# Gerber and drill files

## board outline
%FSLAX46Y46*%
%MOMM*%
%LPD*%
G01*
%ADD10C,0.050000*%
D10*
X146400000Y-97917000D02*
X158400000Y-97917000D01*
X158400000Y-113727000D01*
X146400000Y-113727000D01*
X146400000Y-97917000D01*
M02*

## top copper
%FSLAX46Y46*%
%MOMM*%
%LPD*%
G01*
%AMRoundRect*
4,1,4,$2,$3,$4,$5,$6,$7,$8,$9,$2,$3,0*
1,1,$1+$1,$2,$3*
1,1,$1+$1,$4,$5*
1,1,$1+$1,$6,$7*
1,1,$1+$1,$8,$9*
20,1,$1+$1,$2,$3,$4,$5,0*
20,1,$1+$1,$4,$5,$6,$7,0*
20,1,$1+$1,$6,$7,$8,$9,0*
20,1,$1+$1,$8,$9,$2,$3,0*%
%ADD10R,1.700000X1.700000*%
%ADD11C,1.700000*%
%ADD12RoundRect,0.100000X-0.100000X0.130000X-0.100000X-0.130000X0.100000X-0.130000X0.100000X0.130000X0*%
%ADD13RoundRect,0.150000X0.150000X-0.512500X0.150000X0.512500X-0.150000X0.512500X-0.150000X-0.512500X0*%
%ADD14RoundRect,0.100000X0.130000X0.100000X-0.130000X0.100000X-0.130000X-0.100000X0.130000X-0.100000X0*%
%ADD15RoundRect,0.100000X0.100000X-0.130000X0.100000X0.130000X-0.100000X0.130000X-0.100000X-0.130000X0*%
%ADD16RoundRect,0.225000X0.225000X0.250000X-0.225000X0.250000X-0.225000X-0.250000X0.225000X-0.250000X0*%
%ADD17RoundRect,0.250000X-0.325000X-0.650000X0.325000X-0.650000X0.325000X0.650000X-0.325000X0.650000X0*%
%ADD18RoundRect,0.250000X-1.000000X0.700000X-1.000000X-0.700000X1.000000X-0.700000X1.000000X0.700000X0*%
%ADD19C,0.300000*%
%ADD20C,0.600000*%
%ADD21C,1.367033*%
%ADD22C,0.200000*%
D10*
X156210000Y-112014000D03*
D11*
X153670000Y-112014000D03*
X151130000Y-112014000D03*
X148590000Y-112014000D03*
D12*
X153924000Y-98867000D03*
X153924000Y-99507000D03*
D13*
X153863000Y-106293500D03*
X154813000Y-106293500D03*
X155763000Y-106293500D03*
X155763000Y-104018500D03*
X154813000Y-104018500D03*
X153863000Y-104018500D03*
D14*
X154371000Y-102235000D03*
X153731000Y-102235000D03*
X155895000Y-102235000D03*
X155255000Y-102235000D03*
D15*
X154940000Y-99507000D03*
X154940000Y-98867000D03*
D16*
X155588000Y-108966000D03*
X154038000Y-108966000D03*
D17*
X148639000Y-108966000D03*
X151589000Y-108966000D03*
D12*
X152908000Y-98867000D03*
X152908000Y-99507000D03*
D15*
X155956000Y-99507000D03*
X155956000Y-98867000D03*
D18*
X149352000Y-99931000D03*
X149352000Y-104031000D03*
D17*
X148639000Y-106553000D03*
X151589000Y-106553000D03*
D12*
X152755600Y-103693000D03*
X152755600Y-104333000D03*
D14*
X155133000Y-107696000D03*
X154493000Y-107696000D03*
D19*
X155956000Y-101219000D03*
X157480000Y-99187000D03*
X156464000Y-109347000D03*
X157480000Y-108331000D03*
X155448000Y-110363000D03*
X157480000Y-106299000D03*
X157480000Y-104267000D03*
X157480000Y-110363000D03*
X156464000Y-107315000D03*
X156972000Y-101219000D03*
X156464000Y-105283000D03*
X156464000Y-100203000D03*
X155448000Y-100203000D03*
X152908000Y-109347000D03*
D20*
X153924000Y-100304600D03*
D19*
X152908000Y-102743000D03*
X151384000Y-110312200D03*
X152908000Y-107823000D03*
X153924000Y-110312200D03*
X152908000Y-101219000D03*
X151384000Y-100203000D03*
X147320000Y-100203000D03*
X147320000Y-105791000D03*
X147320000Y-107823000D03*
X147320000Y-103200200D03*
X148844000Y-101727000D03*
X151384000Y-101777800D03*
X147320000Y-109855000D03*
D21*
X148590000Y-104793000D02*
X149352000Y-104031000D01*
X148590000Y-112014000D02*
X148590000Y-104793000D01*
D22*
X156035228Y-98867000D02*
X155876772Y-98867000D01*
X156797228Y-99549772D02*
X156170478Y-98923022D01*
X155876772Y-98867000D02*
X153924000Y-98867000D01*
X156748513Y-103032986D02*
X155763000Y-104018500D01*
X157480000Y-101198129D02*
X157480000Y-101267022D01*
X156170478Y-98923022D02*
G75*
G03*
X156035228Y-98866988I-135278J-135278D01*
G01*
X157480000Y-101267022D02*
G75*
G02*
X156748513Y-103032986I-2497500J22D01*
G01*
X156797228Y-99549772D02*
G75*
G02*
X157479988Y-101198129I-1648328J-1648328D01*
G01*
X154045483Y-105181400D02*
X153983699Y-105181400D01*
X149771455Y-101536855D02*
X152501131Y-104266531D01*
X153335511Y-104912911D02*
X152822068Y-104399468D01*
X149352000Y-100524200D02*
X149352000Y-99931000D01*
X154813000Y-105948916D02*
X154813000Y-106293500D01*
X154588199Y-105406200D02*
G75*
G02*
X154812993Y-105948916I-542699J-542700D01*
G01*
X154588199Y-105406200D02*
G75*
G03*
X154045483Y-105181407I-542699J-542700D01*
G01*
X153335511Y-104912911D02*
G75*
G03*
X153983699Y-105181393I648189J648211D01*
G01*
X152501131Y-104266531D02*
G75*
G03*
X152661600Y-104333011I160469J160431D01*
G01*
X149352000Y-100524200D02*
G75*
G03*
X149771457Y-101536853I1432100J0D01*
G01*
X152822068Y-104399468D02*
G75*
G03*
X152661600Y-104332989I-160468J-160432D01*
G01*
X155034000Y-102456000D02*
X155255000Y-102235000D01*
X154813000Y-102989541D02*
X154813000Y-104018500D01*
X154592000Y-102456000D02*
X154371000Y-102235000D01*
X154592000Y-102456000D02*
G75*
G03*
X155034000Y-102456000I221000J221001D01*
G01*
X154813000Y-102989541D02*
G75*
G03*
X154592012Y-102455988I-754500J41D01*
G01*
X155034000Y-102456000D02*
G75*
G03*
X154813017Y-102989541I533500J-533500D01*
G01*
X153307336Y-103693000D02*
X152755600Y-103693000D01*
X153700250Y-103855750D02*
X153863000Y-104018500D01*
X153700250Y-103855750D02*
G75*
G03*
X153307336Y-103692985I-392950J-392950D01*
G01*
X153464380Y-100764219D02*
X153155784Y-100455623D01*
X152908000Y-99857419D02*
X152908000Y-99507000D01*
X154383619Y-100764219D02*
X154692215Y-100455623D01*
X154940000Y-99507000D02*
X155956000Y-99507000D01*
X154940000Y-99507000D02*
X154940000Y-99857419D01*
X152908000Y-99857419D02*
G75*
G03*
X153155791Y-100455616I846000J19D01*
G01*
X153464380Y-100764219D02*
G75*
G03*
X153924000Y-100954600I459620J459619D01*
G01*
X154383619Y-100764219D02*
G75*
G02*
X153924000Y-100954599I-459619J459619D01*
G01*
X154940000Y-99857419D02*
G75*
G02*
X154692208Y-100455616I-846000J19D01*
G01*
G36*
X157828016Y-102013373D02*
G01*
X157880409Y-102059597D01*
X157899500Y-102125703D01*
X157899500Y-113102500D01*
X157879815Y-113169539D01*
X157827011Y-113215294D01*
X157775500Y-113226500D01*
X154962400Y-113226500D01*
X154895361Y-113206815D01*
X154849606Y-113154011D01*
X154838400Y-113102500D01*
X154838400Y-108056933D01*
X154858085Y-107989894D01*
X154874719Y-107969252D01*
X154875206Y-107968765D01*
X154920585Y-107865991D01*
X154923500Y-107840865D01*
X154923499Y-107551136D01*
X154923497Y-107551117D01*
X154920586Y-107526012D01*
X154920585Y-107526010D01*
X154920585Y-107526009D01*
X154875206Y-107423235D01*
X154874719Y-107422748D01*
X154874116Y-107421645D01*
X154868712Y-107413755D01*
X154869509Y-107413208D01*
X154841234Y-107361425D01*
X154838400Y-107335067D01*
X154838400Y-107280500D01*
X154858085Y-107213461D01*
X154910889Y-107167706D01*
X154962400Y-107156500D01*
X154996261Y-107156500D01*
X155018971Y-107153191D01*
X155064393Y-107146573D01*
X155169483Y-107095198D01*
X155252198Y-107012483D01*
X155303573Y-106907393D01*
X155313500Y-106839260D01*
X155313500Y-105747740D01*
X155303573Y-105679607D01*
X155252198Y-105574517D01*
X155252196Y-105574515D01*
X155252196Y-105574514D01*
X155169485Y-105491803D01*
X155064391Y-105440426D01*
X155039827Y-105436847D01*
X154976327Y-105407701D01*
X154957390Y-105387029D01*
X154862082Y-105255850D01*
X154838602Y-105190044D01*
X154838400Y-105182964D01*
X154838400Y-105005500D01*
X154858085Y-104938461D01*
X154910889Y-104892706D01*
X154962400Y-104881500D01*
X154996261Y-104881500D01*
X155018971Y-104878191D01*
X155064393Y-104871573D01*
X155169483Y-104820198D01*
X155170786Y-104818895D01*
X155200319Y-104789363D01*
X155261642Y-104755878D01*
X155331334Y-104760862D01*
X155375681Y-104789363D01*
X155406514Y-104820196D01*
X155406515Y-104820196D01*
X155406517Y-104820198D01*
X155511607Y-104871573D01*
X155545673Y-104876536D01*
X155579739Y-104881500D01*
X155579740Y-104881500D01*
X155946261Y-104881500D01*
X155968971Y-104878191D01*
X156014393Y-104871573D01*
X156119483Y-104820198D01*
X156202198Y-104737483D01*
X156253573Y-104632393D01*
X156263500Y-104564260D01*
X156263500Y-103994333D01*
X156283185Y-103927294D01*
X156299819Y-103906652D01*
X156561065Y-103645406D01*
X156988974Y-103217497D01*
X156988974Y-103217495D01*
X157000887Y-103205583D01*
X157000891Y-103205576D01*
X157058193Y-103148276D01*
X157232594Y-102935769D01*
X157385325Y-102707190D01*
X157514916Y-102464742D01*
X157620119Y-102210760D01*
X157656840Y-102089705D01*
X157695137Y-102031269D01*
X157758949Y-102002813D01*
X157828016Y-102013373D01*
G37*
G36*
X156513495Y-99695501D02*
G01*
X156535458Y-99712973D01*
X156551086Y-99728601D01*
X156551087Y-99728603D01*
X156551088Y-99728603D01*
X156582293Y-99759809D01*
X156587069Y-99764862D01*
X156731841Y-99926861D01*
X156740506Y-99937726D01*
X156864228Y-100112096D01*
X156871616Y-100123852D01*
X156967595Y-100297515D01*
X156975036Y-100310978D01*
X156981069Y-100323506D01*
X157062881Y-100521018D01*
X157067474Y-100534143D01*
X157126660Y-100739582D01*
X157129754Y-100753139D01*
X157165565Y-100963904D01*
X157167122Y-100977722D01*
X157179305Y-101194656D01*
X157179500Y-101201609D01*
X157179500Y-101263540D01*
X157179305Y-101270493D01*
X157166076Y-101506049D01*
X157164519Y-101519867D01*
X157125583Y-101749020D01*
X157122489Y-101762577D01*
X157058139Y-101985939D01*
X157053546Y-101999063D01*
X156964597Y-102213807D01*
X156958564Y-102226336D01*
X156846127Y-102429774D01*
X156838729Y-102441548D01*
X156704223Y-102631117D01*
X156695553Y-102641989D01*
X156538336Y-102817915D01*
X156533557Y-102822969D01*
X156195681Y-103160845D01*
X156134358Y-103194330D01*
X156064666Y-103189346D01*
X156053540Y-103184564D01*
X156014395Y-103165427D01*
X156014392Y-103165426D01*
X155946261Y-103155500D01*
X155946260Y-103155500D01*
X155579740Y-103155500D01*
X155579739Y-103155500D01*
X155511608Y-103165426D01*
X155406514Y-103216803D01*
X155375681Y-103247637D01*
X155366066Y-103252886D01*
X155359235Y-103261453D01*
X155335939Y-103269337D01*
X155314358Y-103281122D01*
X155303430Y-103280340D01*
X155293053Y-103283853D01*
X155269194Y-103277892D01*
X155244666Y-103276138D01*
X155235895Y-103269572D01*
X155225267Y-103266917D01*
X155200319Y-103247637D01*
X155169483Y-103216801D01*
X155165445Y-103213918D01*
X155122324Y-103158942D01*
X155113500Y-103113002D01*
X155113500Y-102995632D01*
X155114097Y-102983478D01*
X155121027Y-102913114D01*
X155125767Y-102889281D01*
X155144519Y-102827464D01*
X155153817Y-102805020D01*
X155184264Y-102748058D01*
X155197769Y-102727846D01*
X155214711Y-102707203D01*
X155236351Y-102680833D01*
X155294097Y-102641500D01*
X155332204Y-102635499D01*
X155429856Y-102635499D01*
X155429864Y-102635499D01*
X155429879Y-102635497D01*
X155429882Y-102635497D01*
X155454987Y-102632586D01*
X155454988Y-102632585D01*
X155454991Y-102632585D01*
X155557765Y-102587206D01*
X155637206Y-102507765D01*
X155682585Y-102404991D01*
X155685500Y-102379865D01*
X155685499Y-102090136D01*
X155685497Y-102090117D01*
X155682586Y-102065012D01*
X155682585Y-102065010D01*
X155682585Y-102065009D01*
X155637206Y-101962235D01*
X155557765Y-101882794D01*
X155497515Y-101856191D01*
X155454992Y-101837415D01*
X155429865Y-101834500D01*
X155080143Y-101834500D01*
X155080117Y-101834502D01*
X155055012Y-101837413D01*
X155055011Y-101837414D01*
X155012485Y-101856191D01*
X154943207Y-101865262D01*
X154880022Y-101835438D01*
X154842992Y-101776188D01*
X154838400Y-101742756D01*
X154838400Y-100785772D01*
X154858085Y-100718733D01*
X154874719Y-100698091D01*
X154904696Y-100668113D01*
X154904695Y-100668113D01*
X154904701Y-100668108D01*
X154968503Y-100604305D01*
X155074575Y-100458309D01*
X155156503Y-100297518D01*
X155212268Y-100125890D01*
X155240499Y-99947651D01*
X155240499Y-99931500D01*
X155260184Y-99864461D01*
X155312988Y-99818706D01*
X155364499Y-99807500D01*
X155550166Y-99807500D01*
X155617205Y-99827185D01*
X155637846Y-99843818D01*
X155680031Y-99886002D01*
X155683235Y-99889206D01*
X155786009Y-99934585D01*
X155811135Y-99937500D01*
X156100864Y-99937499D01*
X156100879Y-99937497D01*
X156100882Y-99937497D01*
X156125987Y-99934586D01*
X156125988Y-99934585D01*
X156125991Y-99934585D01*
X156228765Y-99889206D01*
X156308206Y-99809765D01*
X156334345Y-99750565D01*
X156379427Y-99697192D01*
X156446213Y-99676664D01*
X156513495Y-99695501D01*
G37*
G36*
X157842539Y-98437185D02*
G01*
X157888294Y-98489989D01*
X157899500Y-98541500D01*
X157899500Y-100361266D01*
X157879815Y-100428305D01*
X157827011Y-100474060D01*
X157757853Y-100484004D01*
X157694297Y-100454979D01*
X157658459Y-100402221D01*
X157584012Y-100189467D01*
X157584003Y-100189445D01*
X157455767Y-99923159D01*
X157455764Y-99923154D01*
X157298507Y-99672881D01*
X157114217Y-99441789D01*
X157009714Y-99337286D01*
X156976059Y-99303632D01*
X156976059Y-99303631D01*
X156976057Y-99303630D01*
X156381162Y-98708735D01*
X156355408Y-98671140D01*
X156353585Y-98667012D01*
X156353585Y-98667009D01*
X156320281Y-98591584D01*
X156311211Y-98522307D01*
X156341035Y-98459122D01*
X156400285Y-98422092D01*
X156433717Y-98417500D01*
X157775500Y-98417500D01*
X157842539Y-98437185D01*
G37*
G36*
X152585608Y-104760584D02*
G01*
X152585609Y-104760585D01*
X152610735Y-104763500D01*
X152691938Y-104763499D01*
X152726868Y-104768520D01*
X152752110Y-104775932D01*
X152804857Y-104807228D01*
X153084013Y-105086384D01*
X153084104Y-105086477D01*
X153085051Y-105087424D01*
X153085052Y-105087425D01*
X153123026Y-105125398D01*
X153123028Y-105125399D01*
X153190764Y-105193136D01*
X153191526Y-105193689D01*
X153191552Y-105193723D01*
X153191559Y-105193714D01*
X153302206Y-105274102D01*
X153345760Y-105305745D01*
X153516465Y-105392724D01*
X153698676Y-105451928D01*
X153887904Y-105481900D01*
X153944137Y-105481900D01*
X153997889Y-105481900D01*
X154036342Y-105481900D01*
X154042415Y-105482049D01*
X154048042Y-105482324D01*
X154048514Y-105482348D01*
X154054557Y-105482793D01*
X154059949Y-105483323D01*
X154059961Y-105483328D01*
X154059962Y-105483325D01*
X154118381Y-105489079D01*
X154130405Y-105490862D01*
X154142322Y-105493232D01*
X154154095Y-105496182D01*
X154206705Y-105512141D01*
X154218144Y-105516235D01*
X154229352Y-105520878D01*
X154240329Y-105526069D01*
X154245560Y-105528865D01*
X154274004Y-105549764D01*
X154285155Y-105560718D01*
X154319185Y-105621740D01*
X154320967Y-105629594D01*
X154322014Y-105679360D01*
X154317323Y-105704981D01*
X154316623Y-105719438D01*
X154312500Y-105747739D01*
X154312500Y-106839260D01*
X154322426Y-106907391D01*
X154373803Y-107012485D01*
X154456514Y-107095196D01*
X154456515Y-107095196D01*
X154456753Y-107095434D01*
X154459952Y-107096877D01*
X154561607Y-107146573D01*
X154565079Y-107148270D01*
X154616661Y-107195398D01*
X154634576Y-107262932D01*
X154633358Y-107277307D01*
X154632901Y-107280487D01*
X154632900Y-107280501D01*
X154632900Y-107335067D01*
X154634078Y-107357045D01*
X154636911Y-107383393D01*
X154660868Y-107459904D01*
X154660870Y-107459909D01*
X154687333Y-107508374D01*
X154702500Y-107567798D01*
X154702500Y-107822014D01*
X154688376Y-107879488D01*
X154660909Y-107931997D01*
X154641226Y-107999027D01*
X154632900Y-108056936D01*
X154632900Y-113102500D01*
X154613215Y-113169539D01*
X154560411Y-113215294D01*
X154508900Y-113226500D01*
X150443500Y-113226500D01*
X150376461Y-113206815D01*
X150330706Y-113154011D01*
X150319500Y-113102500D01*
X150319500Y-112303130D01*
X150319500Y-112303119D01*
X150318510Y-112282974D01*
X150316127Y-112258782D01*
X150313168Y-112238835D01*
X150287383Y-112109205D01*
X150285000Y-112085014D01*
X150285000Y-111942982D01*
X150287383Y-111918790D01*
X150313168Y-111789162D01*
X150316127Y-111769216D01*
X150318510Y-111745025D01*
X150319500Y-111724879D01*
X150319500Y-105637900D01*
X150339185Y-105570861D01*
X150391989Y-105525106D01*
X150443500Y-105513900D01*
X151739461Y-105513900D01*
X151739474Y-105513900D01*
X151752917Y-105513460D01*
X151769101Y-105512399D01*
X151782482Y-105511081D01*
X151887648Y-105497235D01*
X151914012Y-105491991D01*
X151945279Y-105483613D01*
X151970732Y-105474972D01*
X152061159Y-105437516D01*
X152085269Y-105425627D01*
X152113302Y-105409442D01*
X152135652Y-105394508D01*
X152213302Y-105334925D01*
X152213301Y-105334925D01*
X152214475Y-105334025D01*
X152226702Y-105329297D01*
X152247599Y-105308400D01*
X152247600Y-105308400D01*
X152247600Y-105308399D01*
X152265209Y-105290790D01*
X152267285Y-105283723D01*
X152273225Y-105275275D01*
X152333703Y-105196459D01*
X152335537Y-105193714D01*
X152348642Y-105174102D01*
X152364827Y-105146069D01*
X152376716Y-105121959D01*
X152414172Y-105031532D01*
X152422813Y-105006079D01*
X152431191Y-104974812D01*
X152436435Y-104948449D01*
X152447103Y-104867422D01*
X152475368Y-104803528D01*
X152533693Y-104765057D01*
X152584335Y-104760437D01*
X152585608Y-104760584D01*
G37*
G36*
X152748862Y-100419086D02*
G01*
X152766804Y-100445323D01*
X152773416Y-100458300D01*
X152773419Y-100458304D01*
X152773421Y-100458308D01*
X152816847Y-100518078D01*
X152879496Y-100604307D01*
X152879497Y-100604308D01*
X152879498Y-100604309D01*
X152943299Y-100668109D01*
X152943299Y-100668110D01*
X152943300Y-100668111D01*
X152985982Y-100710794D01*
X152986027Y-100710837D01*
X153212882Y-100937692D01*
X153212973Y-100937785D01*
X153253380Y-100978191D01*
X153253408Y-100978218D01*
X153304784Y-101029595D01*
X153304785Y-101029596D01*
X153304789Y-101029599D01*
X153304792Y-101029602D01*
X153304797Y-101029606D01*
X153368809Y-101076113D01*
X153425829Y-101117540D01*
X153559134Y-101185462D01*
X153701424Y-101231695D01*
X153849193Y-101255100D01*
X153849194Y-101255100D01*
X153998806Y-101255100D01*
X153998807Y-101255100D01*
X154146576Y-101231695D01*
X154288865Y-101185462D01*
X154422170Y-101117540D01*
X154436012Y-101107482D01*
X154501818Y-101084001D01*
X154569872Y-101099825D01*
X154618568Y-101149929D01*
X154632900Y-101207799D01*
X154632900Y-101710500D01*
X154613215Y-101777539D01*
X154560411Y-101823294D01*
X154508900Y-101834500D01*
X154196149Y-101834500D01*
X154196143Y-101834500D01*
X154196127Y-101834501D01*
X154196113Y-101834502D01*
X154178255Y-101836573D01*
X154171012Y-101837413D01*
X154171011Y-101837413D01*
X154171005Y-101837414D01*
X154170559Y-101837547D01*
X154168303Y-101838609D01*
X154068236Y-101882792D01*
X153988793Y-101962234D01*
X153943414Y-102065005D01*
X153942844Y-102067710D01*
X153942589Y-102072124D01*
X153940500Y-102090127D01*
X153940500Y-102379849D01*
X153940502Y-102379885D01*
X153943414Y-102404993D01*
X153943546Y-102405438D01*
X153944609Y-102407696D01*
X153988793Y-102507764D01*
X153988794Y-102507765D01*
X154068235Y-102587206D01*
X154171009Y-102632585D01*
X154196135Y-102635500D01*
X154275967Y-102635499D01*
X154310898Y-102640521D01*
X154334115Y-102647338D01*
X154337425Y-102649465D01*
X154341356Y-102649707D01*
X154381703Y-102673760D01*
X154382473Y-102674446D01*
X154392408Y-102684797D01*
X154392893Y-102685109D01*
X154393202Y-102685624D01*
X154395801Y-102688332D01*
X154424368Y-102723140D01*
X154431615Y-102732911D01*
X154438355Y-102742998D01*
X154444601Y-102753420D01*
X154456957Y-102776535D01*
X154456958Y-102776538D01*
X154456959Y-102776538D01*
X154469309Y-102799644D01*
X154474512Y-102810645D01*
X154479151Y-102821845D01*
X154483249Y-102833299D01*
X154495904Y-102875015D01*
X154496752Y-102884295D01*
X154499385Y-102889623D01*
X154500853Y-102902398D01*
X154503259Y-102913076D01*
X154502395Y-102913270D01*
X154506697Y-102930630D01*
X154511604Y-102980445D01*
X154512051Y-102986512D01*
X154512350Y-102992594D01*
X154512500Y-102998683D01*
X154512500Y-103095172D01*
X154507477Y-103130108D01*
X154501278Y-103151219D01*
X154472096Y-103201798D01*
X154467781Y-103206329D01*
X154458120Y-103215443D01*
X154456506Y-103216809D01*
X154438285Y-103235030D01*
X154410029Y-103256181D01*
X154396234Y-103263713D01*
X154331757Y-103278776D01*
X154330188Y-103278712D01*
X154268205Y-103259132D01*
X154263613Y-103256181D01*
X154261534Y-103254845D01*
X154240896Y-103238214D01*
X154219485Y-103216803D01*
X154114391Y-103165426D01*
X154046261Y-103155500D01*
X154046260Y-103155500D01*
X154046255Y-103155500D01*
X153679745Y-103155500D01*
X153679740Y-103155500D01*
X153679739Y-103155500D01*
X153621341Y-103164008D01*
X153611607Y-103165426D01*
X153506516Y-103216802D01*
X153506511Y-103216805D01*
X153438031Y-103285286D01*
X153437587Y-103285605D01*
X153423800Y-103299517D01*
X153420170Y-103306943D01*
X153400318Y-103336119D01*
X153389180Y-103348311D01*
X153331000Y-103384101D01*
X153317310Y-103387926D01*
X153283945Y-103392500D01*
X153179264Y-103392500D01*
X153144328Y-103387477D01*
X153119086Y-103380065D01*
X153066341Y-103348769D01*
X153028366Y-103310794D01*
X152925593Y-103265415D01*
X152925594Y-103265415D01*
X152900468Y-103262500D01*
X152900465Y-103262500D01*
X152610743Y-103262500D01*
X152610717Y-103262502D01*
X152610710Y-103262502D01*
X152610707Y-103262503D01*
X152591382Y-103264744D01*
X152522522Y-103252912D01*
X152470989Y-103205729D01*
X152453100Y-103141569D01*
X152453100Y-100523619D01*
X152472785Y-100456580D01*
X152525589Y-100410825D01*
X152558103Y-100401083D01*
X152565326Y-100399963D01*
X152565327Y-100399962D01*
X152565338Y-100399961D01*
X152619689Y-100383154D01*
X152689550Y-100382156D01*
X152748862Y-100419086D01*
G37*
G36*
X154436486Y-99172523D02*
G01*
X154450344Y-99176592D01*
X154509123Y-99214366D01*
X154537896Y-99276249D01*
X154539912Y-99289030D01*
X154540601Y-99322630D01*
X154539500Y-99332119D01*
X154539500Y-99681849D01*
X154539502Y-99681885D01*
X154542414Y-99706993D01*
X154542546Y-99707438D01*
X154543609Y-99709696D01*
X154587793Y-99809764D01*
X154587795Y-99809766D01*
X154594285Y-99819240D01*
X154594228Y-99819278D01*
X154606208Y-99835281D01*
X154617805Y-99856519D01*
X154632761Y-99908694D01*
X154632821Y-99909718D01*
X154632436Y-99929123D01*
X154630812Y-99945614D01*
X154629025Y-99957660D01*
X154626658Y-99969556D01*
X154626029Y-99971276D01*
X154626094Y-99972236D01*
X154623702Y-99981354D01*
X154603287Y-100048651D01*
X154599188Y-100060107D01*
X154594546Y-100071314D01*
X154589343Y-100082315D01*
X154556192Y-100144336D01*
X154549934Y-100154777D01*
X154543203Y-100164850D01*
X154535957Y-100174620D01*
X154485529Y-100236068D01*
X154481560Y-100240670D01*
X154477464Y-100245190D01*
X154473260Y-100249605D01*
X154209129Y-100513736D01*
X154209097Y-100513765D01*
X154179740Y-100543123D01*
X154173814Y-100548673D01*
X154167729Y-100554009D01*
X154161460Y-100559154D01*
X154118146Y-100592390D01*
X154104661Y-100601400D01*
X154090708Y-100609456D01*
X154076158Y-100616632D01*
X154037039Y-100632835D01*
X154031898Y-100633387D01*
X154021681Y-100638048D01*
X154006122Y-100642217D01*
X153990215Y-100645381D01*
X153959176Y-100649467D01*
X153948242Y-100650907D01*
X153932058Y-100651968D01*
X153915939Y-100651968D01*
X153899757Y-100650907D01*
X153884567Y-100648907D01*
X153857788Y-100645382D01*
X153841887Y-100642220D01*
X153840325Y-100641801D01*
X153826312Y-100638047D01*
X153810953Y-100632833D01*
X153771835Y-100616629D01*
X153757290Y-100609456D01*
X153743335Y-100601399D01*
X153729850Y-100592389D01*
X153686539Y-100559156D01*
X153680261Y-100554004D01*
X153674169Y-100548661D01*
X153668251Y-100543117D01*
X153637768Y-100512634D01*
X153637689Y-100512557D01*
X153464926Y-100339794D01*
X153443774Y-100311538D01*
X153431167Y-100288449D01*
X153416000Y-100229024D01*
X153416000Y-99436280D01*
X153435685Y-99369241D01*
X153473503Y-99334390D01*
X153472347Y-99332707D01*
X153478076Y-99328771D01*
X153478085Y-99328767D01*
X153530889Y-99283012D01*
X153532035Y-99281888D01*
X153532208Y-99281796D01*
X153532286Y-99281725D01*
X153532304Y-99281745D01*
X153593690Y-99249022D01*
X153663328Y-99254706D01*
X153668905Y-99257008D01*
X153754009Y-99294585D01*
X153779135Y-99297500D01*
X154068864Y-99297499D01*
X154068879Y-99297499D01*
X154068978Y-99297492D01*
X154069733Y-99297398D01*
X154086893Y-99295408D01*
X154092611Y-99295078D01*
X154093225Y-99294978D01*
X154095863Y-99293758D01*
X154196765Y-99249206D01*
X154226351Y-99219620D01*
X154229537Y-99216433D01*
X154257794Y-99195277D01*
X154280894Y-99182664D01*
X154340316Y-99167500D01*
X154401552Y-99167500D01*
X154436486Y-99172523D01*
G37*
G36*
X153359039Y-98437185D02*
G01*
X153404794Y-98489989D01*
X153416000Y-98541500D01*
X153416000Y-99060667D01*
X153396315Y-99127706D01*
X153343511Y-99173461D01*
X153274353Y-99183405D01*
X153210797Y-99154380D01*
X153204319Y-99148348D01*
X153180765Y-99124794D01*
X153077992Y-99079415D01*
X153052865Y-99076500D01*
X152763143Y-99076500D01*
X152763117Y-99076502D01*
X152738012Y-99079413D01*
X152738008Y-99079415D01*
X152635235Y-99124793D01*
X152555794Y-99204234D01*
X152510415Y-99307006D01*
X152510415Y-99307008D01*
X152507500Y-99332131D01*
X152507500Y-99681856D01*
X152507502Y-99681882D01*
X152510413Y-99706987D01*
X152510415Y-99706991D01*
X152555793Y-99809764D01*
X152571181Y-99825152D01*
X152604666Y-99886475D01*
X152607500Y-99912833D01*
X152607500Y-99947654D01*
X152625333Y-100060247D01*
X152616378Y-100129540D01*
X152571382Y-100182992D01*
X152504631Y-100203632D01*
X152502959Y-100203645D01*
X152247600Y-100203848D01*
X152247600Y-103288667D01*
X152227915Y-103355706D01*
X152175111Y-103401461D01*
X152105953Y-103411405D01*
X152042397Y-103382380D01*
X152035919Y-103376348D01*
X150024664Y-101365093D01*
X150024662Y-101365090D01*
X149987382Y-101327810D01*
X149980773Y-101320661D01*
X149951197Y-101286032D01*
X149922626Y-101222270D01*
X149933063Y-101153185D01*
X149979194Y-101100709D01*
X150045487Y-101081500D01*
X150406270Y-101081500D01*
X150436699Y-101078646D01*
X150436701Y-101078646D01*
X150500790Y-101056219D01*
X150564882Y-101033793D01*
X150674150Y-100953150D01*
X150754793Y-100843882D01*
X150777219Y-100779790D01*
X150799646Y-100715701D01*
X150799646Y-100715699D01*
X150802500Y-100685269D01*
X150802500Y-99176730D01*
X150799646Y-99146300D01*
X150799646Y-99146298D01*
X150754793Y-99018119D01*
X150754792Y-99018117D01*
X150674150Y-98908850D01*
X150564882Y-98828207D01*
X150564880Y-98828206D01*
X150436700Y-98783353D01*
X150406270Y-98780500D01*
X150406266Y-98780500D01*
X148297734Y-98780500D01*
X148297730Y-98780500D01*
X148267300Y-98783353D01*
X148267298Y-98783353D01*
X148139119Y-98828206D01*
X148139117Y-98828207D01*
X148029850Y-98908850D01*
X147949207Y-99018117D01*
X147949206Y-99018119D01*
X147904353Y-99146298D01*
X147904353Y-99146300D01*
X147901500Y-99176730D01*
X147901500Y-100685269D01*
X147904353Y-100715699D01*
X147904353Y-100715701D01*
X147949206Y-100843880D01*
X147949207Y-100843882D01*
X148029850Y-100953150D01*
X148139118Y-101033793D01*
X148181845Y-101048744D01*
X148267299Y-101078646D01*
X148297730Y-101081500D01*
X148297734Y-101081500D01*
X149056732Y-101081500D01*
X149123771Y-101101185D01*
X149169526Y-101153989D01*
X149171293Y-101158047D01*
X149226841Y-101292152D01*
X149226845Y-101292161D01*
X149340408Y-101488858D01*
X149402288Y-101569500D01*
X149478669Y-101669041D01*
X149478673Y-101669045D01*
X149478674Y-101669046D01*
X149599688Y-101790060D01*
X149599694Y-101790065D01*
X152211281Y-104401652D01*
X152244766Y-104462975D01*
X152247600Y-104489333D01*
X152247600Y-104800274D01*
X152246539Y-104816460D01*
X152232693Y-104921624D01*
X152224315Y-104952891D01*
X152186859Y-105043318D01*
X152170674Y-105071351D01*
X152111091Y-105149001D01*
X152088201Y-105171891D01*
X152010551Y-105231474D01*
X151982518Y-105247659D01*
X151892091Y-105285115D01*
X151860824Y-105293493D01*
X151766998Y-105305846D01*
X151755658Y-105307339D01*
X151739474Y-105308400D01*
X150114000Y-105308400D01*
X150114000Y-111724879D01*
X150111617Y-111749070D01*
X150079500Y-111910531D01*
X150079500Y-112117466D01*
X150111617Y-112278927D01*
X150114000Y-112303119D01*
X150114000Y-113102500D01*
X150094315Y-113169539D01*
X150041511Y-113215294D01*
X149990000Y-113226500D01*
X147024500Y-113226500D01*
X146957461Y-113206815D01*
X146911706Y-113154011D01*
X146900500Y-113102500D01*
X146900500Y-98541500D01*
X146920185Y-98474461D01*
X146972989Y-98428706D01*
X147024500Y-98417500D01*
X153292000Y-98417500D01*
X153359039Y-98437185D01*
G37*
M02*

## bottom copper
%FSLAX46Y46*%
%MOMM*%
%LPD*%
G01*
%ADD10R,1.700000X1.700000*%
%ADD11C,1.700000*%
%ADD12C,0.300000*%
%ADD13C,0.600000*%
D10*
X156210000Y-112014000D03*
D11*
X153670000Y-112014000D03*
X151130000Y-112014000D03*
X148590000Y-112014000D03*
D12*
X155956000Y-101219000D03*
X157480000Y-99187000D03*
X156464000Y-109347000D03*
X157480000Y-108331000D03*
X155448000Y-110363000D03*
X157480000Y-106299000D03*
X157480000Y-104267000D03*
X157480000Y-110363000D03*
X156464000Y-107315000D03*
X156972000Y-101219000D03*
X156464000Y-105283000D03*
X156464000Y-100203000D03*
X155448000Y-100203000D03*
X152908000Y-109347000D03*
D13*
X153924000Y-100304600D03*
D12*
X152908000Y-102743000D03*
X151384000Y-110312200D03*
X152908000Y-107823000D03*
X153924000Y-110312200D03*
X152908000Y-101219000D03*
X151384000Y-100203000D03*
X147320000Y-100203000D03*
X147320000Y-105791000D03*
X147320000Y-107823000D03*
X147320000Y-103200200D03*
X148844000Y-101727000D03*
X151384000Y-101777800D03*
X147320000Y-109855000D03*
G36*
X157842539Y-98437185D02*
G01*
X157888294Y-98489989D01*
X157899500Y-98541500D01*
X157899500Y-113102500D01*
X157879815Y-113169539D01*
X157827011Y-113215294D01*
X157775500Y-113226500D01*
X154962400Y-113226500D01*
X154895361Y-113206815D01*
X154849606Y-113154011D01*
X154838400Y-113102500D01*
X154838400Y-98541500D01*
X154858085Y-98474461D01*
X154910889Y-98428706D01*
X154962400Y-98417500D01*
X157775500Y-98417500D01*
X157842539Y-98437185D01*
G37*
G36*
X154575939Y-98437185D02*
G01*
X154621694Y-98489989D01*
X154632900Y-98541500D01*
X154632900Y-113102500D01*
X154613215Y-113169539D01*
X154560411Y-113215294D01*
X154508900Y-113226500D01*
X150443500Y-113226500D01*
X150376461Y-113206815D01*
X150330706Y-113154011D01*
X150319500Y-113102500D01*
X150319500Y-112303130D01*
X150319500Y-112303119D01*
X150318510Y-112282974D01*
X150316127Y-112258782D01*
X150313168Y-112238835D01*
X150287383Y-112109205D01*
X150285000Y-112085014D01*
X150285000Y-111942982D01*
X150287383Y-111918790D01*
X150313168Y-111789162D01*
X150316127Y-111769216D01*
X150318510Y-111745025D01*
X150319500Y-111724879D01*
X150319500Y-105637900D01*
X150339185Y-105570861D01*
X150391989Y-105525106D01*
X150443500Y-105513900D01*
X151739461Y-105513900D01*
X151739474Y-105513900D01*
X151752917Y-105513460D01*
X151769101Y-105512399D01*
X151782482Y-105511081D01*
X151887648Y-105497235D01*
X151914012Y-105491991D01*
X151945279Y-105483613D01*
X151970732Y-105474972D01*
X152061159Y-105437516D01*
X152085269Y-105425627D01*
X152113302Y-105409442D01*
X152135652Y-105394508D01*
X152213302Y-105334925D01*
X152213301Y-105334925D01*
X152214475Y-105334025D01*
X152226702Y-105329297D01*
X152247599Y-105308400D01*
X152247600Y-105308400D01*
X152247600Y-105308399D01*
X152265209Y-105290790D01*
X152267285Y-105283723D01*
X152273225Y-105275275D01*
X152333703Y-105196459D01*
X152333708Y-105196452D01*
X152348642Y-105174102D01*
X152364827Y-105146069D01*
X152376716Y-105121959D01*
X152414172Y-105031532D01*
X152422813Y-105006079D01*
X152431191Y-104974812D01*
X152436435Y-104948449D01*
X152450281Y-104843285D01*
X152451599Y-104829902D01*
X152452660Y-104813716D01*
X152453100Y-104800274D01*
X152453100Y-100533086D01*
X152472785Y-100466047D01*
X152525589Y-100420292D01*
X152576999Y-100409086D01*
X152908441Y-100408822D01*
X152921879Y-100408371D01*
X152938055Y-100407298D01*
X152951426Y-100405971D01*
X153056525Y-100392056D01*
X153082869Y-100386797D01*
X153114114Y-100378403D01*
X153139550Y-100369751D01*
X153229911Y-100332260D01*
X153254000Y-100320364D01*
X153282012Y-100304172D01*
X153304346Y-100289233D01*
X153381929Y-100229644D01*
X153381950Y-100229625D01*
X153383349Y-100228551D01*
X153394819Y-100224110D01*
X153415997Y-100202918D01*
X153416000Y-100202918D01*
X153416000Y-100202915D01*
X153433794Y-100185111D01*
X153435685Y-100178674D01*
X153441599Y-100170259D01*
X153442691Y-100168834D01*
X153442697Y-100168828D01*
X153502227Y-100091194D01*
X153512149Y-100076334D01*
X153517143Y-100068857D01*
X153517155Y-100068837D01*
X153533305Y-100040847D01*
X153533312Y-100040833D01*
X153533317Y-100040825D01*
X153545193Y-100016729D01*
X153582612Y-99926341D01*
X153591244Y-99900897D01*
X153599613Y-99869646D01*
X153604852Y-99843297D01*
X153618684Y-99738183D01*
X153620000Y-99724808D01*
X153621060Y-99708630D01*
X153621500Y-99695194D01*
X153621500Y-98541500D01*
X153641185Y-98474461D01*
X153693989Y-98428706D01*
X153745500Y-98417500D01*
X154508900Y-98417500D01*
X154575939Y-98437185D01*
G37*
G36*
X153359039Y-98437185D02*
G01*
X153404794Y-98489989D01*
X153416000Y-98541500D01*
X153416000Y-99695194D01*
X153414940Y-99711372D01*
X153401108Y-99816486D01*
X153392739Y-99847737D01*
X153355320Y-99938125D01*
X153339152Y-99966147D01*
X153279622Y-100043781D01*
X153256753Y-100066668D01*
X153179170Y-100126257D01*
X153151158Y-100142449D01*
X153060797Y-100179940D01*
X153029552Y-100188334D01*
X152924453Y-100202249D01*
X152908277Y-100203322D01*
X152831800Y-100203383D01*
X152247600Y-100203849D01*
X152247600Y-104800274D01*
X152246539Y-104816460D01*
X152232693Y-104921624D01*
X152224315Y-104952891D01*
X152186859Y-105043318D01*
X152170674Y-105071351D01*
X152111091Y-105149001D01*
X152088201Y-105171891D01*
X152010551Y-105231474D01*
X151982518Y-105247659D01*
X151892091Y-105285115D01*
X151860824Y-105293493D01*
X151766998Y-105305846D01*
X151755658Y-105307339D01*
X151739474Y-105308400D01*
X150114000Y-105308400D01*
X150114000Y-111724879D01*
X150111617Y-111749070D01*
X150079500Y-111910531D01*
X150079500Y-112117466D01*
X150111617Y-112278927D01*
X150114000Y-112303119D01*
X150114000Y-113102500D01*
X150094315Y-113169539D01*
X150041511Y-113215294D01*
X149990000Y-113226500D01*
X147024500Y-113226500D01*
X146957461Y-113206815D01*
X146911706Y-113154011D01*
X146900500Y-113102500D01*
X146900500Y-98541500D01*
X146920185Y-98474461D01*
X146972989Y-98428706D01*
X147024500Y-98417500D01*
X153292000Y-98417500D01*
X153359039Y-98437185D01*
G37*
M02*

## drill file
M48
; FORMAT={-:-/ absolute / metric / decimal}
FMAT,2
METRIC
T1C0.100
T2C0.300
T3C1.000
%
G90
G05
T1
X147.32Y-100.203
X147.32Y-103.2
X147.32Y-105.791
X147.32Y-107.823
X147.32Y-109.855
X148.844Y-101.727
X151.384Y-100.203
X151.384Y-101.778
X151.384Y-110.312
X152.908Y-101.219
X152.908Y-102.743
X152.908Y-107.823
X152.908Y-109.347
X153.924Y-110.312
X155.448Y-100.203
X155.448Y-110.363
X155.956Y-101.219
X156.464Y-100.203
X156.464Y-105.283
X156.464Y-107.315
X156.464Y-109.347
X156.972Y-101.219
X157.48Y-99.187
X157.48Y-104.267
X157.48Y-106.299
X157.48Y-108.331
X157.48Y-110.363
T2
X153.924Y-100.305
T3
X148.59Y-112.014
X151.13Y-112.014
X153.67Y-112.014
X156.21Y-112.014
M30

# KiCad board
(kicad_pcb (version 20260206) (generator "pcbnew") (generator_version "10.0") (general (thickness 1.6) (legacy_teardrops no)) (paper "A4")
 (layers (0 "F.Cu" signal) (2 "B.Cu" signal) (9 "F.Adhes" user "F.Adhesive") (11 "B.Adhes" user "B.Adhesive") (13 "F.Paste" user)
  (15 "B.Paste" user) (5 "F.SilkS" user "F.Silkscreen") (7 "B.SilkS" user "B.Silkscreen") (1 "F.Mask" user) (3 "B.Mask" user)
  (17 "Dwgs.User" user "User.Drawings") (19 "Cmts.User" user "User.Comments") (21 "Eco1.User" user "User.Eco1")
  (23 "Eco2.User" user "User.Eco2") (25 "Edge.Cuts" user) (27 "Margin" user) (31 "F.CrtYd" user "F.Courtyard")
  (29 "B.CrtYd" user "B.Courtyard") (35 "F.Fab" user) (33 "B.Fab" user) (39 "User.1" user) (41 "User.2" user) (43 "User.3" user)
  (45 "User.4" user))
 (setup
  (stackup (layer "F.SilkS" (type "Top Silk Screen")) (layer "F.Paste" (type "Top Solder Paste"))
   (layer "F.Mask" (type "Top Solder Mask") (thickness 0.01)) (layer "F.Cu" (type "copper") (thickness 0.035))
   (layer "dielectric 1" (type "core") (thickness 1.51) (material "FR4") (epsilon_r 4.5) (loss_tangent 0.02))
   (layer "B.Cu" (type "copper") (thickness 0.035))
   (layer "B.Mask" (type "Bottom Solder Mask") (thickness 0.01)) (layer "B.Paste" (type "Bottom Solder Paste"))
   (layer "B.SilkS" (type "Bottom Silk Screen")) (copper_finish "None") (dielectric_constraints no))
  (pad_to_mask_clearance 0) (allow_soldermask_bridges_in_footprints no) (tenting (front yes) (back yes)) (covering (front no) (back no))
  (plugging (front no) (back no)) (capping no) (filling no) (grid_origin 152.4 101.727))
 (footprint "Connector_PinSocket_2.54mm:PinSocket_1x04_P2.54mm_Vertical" (layer "F.Cu") (at 156.21 112.014 -90)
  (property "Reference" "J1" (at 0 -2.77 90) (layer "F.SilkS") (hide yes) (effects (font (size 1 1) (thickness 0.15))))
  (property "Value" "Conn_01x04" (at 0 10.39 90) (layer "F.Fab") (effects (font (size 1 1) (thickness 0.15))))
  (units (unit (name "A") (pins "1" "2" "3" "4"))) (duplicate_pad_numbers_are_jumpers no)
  (pad "1" thru_hole rect (at 0 0 270) (size 1.7 1.7) (drill 1) (layers "*.Cu" "*.Mask") (remove_unused_layers no) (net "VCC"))
  (pad "2" thru_hole circle (at 0 2.54 270) (size 1.7 1.7) (drill 1) (layers "*.Cu" "*.Mask") (remove_unused_layers no) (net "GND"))
  (pad "3" thru_hole circle (at 0 5.08 270) (size 1.7 1.7) (drill 1) (layers "*.Cu" "*.Mask") (remove_unused_layers no) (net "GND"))
  (pad "4" thru_hole circle (at 0 7.62 270) (size 1.7 1.7) (drill 1) (layers "*.Cu" "*.Mask") (remove_unused_layers no) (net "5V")))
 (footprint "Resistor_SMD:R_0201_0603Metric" (layer "F.Cu") (at 153.924 99.187 -90)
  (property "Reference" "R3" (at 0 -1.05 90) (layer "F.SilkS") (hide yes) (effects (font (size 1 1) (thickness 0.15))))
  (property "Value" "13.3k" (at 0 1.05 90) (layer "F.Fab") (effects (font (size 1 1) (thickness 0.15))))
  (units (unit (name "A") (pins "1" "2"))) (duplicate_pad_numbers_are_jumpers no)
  (pad "" smd roundrect (at -0.345 0 270) (size 0.318 0.36) (layers "F.Paste") (roundrect_rratio 0.25))
  (pad "" smd roundrect (at 0.345 0 270) (size 0.318 0.36) (layers "F.Paste") (roundrect_rratio 0.25))
  (pad "1" smd roundrect (at -0.32 0 270) (size 0.46 0.4) (layers "F.Cu" "F.Mask") (roundrect_rratio 0.25) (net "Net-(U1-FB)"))
  (pad "2" smd roundrect (at 0.32 0 270) (size 0.46 0.4) (layers "F.Cu" "F.Mask") (roundrect_rratio 0.25) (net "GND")))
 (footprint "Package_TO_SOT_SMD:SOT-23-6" (layer "F.Cu") (at 154.813 105.156 90)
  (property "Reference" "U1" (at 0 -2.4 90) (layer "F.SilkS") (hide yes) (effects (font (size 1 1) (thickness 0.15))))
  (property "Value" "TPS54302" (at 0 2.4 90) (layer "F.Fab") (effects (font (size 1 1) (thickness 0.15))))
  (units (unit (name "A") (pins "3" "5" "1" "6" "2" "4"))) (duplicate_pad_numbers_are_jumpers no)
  (pad "1" smd roundrect (at -1.1375 -0.95 90) (size 1.325 0.6) (layers "F.Cu" "F.Mask" "F.Paste") (roundrect_rratio 0.25) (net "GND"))
  (pad "2" smd roundrect (at -1.1375 0 90) (size 1.325 0.6) (layers "F.Cu" "F.Mask" "F.Paste") (roundrect_rratio 0.25) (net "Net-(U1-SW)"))
  (pad "3" smd roundrect (at -1.1375 0.95 90) (size 1.325 0.6) (layers "F.Cu" "F.Mask" "F.Paste") (roundrect_rratio 0.25) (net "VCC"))
  (pad "4" smd roundrect (at 1.1375 0.95 90) (size 1.325 0.6) (layers "F.Cu" "F.Mask" "F.Paste") (roundrect_rratio 0.25) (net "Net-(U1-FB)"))
  (pad "5" smd roundrect (at 1.1375 0 90) (size 1.325 0.6) (layers "F.Cu" "F.Mask" "F.Paste") (roundrect_rratio 0.25) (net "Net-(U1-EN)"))
  (pad "6" smd roundrect (at 1.1375 -0.95 90) (size 1.325 0.6) (layers "F.Cu" "F.Mask" "F.Paste") (roundrect_rratio 0.25)
   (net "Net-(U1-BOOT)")))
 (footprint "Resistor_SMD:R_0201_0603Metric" (layer "F.Cu") (at 154.051 102.235 180)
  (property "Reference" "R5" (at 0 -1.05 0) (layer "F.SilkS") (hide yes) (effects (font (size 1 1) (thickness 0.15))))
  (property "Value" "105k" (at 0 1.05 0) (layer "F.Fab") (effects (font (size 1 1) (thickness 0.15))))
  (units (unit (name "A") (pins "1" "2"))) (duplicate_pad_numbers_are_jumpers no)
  (pad "" smd roundrect (at -0.345 0 180) (size 0.318 0.36) (layers "F.Paste") (roundrect_rratio 0.25))
  (pad "" smd roundrect (at 0.345 0 180) (size 0.318 0.36) (layers "F.Paste") (roundrect_rratio 0.25))
  (pad "1" smd roundrect (at -0.32 0 180) (size 0.46 0.4) (layers "F.Cu" "F.Mask") (roundrect_rratio 0.25) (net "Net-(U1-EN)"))
  (pad "2" smd roundrect (at 0.32 0 180) (size 0.46 0.4) (layers "F.Cu" "F.Mask") (roundrect_rratio 0.25) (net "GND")))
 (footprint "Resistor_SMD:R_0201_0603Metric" (layer "F.Cu") (at 155.575 102.235 180)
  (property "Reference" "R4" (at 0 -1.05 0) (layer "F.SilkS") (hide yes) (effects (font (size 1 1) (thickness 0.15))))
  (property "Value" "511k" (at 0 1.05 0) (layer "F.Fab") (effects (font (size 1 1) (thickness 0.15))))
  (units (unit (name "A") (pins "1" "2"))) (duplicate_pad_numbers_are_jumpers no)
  (pad "" smd roundrect (at -0.345 0 180) (size 0.318 0.36) (layers "F.Paste") (roundrect_rratio 0.25))
  (pad "" smd roundrect (at 0.345 0 180) (size 0.318 0.36) (layers "F.Paste") (roundrect_rratio 0.25))
  (pad "1" smd roundrect (at -0.32 0 180) (size 0.46 0.4) (layers "F.Cu" "F.Mask") (roundrect_rratio 0.25) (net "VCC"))
  (pad "2" smd roundrect (at 0.32 0 180) (size 0.46 0.4) (layers "F.Cu" "F.Mask") (roundrect_rratio 0.25) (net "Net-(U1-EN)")))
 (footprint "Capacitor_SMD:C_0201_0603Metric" (layer "F.Cu") (at 154.94 99.187 90)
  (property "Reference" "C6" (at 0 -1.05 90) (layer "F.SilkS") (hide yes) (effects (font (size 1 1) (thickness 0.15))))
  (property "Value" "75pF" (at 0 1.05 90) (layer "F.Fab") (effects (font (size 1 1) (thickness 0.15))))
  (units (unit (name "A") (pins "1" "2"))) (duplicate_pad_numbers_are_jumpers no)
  (pad "" smd roundrect (at -0.345 0 90) (size 0.318 0.36) (layers "F.Paste") (roundrect_rratio 0.25))
  (pad "" smd roundrect (at 0.345 0 90) (size 0.318 0.36) (layers "F.Paste") (roundrect_rratio 0.25))
  (pad "1" smd roundrect (at -0.32 0 90) (size 0.46 0.4) (layers "F.Cu" "F.Mask") (roundrect_rratio 0.25) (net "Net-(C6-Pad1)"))
  (pad "2" smd roundrect (at 0.32 0 90) (size 0.46 0.4) (layers "F.Cu" "F.Mask") (roundrect_rratio 0.25) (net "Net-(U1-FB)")))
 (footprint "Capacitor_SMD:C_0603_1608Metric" (layer "F.Cu") (at 154.813 108.966 180)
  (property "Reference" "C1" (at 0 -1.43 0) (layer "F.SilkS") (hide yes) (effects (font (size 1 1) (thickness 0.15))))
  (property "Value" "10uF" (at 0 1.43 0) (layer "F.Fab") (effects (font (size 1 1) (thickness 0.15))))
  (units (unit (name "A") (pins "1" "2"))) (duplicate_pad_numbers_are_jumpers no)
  (pad "1" smd roundrect (at -0.775 0 180) (size 0.9 0.95) (layers "F.Cu" "F.Mask" "F.Paste") (roundrect_rratio 0.25) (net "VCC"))
  (pad "2" smd roundrect (at 0.775 0 180) (size 0.9 0.95) (layers "F.Cu" "F.Mask" "F.Paste") (roundrect_rratio 0.25) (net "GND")))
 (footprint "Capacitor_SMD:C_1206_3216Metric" (layer "F.Cu") (at 150.114 108.966)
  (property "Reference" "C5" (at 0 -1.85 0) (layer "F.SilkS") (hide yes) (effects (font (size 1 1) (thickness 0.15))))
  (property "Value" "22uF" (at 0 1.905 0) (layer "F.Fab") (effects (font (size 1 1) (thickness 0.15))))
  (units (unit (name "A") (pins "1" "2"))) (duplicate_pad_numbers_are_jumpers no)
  (pad "1" smd roundrect (at -1.475 0) (size 1.15 1.8) (layers "F.Cu" "F.Mask" "F.Paste") (roundrect_rratio 0.217391) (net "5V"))
  (pad "2" smd roundrect (at 1.475 0) (size 1.15 1.8) (layers "F.Cu" "F.Mask" "F.Paste") (roundrect_rratio 0.217391) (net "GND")))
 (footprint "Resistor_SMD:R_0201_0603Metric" (layer "F.Cu") (at 152.908 99.187 -90)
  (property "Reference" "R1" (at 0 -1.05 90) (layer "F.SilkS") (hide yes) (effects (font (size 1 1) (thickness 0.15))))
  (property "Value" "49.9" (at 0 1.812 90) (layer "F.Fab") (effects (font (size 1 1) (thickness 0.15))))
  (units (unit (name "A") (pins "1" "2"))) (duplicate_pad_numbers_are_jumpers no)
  (pad "" smd roundrect (at -0.345 0 270) (size 0.318 0.36) (layers "F.Paste") (roundrect_rratio 0.25))
  (pad "" smd roundrect (at 0.345 0 270) (size 0.318 0.36) (layers "F.Paste") (roundrect_rratio 0.25))
  (pad "1" smd roundrect (at -0.32 0 270) (size 0.46 0.4) (layers "F.Cu" "F.Mask") (roundrect_rratio 0.25) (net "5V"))
  (pad "2" smd roundrect (at 0.32 0 270) (size 0.46 0.4) (layers "F.Cu" "F.Mask") (roundrect_rratio 0.25) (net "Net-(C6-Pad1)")))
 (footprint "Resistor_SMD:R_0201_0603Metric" (layer "F.Cu") (at 155.956 99.187 90)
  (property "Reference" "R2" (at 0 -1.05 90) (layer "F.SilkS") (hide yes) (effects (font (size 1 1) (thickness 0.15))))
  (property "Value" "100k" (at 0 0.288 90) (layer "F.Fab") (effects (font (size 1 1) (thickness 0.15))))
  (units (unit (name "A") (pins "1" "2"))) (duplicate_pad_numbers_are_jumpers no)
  (pad "" smd roundrect (at -0.345 0 90) (size 0.318 0.36) (layers "F.Paste") (roundrect_rratio 0.25))
  (pad "" smd roundrect (at 0.345 0 90) (size 0.318 0.36) (layers "F.Paste") (roundrect_rratio 0.25))
  (pad "1" smd roundrect (at -0.32 0 90) (size 0.46 0.4) (layers "F.Cu" "F.Mask") (roundrect_rratio 0.25) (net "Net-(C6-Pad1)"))
  (pad "2" smd roundrect (at 0.32 0 90) (size 0.46 0.4) (layers "F.Cu" "F.Mask") (roundrect_rratio 0.25) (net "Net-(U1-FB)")))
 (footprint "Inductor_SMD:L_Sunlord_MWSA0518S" (layer "F.Cu") (at 149.352 101.981 -90)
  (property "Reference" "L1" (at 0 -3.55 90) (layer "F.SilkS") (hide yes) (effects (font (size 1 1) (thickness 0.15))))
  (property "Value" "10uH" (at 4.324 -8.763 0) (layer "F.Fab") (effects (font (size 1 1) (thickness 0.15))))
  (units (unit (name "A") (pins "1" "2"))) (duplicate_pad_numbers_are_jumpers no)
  (pad "1" smd roundrect (at -2.05 0 270) (size 1.9 2.5) (layers "F.Cu" "F.Mask" "F.Paste") (roundrect_rratio 0.131579) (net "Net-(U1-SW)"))
  (pad "2" smd roundrect (at 2.05 0 270) (size 1.9 2.5) (layers "F.Cu" "F.Mask" "F.Paste") (roundrect_rratio 0.131579) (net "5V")))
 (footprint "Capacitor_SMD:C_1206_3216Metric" (layer "F.Cu") (at 150.114 106.553)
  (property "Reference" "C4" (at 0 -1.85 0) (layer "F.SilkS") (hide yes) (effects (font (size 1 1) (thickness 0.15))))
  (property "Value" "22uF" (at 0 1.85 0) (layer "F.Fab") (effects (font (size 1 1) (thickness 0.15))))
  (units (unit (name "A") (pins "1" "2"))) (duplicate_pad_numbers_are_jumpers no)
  (pad "1" smd roundrect (at -1.475 0) (size 1.15 1.8) (layers "F.Cu" "F.Mask" "F.Paste") (roundrect_rratio 0.217391) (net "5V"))
  (pad "2" smd roundrect (at 1.475 0) (size 1.15 1.8) (layers "F.Cu" "F.Mask" "F.Paste") (roundrect_rratio 0.217391) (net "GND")))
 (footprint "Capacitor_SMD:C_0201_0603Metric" (layer "F.Cu") (at 152.7556 104.013 -90)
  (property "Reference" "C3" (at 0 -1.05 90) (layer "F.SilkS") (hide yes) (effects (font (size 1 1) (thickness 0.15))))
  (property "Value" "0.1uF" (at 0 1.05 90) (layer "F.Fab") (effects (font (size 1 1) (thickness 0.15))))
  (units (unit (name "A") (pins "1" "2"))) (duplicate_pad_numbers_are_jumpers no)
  (pad "" smd roundrect (at -0.345 0 270) (size 0.318 0.36) (layers "F.Paste") (roundrect_rratio 0.25))
  (pad "" smd roundrect (at 0.345 0 270) (size 0.318 0.36) (layers "F.Paste") (roundrect_rratio 0.25))
  (pad "1" smd roundrect (at -0.32 0 270) (size 0.46 0.4) (layers "F.Cu" "F.Mask") (roundrect_rratio 0.25) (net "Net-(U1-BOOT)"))
  (pad "2" smd roundrect (at 0.32 0 270) (size 0.46 0.4) (layers "F.Cu" "F.Mask") (roundrect_rratio 0.25) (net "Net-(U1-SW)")))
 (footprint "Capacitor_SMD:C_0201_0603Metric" (layer "F.Cu") (at 154.813 107.696 180)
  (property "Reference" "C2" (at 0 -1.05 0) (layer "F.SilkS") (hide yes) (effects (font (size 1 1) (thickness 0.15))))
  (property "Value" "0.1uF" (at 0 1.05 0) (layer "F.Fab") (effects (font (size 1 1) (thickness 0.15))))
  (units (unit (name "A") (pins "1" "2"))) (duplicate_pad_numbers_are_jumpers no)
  (pad "" smd roundrect (at -0.345 0 180) (size 0.318 0.36) (layers "F.Paste") (roundrect_rratio 0.25))
  (pad "" smd roundrect (at 0.345 0 180) (size 0.318 0.36) (layers "F.Paste") (roundrect_rratio 0.25))
  (pad "1" smd roundrect (at -0.32 0 180) (size 0.46 0.4) (layers "F.Cu" "F.Mask") (roundrect_rratio 0.25) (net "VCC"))
  (pad "2" smd roundrect (at 0.32 0 180) (size 0.46 0.4) (layers "F.Cu" "F.Mask") (roundrect_rratio 0.25) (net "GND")))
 (gr_rect (start 146.4 97.917) (end 158.4 113.727) (stroke (width 0.05) (type default)) (fill no) (layer "Edge.Cuts"))
 (via (at 155.956 101.219) (size 0.3) (drill 0.1) (layers "F.Cu" "B.Cu") (free yes) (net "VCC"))
 (via (at 157.48 99.187) (size 0.3) (drill 0.1) (layers "F.Cu" "B.Cu") (free yes) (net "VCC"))
 (via (at 156.464 109.347) (size 0.3) (drill 0.1) (layers "F.Cu" "B.Cu") (free yes) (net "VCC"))
 (via (at 157.48 108.331) (size 0.3) (drill 0.1) (layers "F.Cu" "B.Cu") (free yes) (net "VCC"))
 (via (at 155.448 110.363) (size 0.3) (drill 0.1) (layers "F.Cu" "B.Cu") (free yes) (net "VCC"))
 (via (at 157.48 106.299) (size 0.3) (drill 0.1) (layers "F.Cu" "B.Cu") (free yes) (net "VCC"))
 (via (at 157.48 104.267) (size 0.3) (drill 0.1) (layers "F.Cu" "B.Cu") (free yes) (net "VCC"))
 (via (at 157.48 110.363) (size 0.3) (drill 0.1) (layers "F.Cu" "B.Cu") (free yes) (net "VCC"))
 (via (at 156.464 107.315) (size 0.3) (drill 0.1) (layers "F.Cu" "B.Cu") (free yes) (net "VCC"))
 (via (at 156.972 101.219) (size 0.3) (drill 0.1) (layers "F.Cu" "B.Cu") (free yes) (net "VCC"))
 (via (at 156.464 105.283) (size 0.3) (drill 0.1) (layers "F.Cu" "B.Cu") (free yes) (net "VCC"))
 (via (at 156.464 100.203) (size 0.3) (drill 0.1) (layers "F.Cu" "B.Cu") (free yes) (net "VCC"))
 (via (at 155.448 100.203) (size 0.3) (drill 0.1) (layers "F.Cu" "B.Cu") (free yes) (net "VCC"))
 (via (at 152.908 109.347) (size 0.3) (drill 0.1) (layers "F.Cu" "B.Cu") (free yes) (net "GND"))
 (via (at 153.924 100.3046) (size 0.6) (drill 0.3) (layers "F.Cu" "B.Cu") (free yes) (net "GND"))
 (via (at 152.908 102.743) (size 0.3) (drill 0.1) (layers "F.Cu" "B.Cu") (free yes) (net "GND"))
 (via (at 151.384 110.3122) (size 0.3) (drill 0.1) (layers "F.Cu" "B.Cu") (free yes) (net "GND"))
 (via (at 152.908 107.823) (size 0.3) (drill 0.1) (layers "F.Cu" "B.Cu") (free yes) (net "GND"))
 (via (at 153.924 110.3122) (size 0.3) (drill 0.1) (layers "F.Cu" "B.Cu") (free yes) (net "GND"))
 (via (at 152.908 101.219) (size 0.3) (drill 0.1) (layers "F.Cu" "B.Cu") (free yes) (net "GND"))
 (segment (start 148.59 104.793) (end 149.352 104.031) (width 1.367033) (layer "F.Cu") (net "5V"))
 (segment (start 148.59 112.014) (end 148.59 104.793) (width 1.367033) (layer "F.Cu") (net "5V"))
 (via (at 151.384 100.203) (size 0.3) (drill 0.1) (layers "F.Cu" "B.Cu") (free yes) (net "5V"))
 (via (at 147.32 100.203) (size 0.3) (drill 0.1) (layers "F.Cu" "B.Cu") (free yes) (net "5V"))
 (via (at 147.32 105.791) (size 0.3) (drill 0.1) (layers "F.Cu" "B.Cu") (free yes) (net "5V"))
 (via (at 147.32 107.823) (size 0.3) (drill 0.1) (layers "F.Cu" "B.Cu") (free yes) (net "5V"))
 (via (at 147.32 103.2002) (size 0.3) (drill 0.1) (layers "F.Cu" "B.Cu") (free yes) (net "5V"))
 (via (at 148.844 101.727) (size 0.3) (drill 0.1) (layers "F.Cu" "B.Cu") (free yes) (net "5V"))
 (via (at 151.384 101.7778) (size 0.3) (drill 0.1) (layers "F.Cu" "B.Cu") (free yes) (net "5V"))
 (via (at 147.32 109.855) (size 0.3) (drill 0.1) (layers "F.Cu" "B.Cu") (free yes) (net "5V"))
 (segment (start 156.035228 98.867) (end 155.876772 98.867) (width 0.2) (layer "F.Cu") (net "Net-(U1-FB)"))
 (segment (start 156.797228 99.549772) (end 156.170478 98.923022) (width 0.2) (layer "F.Cu") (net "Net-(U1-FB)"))
 (segment (start 155.876772 98.867) (end 153.924 98.867) (width 0.2) (layer "F.Cu") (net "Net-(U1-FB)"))
 (segment (start 156.748513 103.032986) (end 155.763 104.0185) (width 0.2) (layer "F.Cu") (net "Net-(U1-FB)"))
 (segment (start 157.48 101.198129) (end 157.48 101.267022) (width 0.2) (layer "F.Cu") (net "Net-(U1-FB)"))
 (arc (start 156.170478 98.923022) (mid 156.108424 98.881559) (end 156.035228 98.867) (width 0.2) (layer "F.Cu") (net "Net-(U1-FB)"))
 (arc (start 157.48 101.267022) (mid 157.289892 102.222754) (end 156.748513 103.032986) (width 0.2) (layer "F.Cu") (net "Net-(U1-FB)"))
 (arc (start 156.797228 99.549772) (mid 157.302553 100.306044) (end 157.48 101.198129) (width 0.2) (layer "F.Cu") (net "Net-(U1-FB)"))
 (segment (start 154.045483 105.1814) (end 153.983699 105.1814) (width 0.2) (layer "F.Cu") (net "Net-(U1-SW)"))
 (segment (start 149.771455 101.536855) (end 152.501131 104.266531) (width 0.2) (layer "F.Cu") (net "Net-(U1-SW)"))
 (segment (start 153.335511 104.912911) (end 152.822068 104.399468) (width 0.2) (layer "F.Cu") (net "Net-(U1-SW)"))
 (segment (start 149.352 100.5242) (end 149.352 99.931) (width 0.2) (layer "F.Cu") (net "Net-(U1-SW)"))
 (segment (start 154.813 105.948916) (end 154.813 106.2935) (width 0.2) (layer "F.Cu") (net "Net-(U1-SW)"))
 (arc (start 154.588199 105.4062) (mid 154.754576 105.6552) (end 154.813 105.948916) (width 0.2) (layer "F.Cu") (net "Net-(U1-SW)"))
 (arc (start 154.588199 105.4062) (mid 154.339198 105.239823) (end 154.045483 105.1814) (width 0.2) (layer "F.Cu") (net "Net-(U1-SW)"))
 (arc (start 153.335511 104.912911) (mid 153.632902 105.111621) (end 153.983699 105.1814) (width 0.2) (layer "F.Cu") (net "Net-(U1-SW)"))
 (arc (start 152.501131 104.266531) (mid 152.574755 104.315725) (end 152.6616 104.333) (width 0.2) (layer "F.Cu") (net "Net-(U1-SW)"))
 (arc (start 149.352 100.5242) (mid 149.461012 101.072245) (end 149.771455 101.536855) (width 0.2) (layer "F.Cu") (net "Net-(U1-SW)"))
 (arc (start 152.822068 104.399468) (mid 152.748444 104.350274) (end 152.6616 104.333) (width 0.2) (layer "F.Cu") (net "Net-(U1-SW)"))
 (segment (start 155.034 102.456) (end 155.255 102.235) (width 0.2) (layer "F.Cu") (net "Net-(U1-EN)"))
 (segment (start 154.813 102.989541) (end 154.813 104.0185) (width 0.2) (layer "F.Cu") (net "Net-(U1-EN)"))
 (segment (start 154.592 102.456) (end 154.371 102.235) (width 0.2) (layer "F.Cu") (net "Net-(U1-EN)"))
 (arc (start 154.592 102.456) (mid 154.813 102.547541) (end 155.034 102.456) (width 0.2) (layer "F.Cu") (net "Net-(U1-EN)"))
 (arc (start 154.813 102.989541) (mid 154.755563 102.70079) (end 154.592 102.456) (width 0.2) (layer "F.Cu") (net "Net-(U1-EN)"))
 (arc (start 155.034 102.456) (mid 154.870436 102.70079) (end 154.813 102.989541) (width 0.2) (layer "F.Cu") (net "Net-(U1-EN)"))
 (segment (start 153.307336 103.693) (end 152.7556 103.693) (width 0.2) (layer "F.Cu") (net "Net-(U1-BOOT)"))
 (segment (start 153.70025 103.85575) (end 153.863 104.0185) (width 0.2) (layer "F.Cu") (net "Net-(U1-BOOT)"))
 (arc (start 153.70025 103.85575) (mid 153.519979 103.735297) (end 153.307336 103.693) (width 0.2) (layer "F.Cu") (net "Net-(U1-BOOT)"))
 (segment (start 153.46438 100.764219) (end 153.155784 100.455623) (width 0.2) (layer "F.Cu") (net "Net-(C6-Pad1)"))
 (segment (start 152.908 99.857419) (end 152.908 99.507) (width 0.2) (layer "F.Cu") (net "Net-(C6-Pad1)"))
 (segment (start 154.383619 100.764219) (end 154.692215 100.455623) (width 0.2) (layer "F.Cu") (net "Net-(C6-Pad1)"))
 (segment (start 154.94 99.507) (end 155.956 99.507) (width 0.2) (layer "F.Cu") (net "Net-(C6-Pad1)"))
 (segment (start 154.94 99.507) (end 154.94 99.857419) (width 0.2) (layer "F.Cu") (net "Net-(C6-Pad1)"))
 (arc (start 152.908 99.857419) (mid 152.972396 100.181164) (end 153.155784 100.455623) (width 0.2) (layer "F.Cu") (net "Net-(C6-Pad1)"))
 (arc (start 153.46438 100.764219) (mid 153.675255 100.905121) (end 153.924 100.9546) (width 0.2) (layer "F.Cu") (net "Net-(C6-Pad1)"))
 (arc (start 154.383619 100.764219) (mid 154.172744 100.905121) (end 153.924 100.9546) (width 0.2) (layer "F.Cu") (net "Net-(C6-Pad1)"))
 (arc (start 154.94 99.857419) (mid 154.875602 100.181164) (end 154.692215 100.455623) (width 0.2) (layer "F.Cu") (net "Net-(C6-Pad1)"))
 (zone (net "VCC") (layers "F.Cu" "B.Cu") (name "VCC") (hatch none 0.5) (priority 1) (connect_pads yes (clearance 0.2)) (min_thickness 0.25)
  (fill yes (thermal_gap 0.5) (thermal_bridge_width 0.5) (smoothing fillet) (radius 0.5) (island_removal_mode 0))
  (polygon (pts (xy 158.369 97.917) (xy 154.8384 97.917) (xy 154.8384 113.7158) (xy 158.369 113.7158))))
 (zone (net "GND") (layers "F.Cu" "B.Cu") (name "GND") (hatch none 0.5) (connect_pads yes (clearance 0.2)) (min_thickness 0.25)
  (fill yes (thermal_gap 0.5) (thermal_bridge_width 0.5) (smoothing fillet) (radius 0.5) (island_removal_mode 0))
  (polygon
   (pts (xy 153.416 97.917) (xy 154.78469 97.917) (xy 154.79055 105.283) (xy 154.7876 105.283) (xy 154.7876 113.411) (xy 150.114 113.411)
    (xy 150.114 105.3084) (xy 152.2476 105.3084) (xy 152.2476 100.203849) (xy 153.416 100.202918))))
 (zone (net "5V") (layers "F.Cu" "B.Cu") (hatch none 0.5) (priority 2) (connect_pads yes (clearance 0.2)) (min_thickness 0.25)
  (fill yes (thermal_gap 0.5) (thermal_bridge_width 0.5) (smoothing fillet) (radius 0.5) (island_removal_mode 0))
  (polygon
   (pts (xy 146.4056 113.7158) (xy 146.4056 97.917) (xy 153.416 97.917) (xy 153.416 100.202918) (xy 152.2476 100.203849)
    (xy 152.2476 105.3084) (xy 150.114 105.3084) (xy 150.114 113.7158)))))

